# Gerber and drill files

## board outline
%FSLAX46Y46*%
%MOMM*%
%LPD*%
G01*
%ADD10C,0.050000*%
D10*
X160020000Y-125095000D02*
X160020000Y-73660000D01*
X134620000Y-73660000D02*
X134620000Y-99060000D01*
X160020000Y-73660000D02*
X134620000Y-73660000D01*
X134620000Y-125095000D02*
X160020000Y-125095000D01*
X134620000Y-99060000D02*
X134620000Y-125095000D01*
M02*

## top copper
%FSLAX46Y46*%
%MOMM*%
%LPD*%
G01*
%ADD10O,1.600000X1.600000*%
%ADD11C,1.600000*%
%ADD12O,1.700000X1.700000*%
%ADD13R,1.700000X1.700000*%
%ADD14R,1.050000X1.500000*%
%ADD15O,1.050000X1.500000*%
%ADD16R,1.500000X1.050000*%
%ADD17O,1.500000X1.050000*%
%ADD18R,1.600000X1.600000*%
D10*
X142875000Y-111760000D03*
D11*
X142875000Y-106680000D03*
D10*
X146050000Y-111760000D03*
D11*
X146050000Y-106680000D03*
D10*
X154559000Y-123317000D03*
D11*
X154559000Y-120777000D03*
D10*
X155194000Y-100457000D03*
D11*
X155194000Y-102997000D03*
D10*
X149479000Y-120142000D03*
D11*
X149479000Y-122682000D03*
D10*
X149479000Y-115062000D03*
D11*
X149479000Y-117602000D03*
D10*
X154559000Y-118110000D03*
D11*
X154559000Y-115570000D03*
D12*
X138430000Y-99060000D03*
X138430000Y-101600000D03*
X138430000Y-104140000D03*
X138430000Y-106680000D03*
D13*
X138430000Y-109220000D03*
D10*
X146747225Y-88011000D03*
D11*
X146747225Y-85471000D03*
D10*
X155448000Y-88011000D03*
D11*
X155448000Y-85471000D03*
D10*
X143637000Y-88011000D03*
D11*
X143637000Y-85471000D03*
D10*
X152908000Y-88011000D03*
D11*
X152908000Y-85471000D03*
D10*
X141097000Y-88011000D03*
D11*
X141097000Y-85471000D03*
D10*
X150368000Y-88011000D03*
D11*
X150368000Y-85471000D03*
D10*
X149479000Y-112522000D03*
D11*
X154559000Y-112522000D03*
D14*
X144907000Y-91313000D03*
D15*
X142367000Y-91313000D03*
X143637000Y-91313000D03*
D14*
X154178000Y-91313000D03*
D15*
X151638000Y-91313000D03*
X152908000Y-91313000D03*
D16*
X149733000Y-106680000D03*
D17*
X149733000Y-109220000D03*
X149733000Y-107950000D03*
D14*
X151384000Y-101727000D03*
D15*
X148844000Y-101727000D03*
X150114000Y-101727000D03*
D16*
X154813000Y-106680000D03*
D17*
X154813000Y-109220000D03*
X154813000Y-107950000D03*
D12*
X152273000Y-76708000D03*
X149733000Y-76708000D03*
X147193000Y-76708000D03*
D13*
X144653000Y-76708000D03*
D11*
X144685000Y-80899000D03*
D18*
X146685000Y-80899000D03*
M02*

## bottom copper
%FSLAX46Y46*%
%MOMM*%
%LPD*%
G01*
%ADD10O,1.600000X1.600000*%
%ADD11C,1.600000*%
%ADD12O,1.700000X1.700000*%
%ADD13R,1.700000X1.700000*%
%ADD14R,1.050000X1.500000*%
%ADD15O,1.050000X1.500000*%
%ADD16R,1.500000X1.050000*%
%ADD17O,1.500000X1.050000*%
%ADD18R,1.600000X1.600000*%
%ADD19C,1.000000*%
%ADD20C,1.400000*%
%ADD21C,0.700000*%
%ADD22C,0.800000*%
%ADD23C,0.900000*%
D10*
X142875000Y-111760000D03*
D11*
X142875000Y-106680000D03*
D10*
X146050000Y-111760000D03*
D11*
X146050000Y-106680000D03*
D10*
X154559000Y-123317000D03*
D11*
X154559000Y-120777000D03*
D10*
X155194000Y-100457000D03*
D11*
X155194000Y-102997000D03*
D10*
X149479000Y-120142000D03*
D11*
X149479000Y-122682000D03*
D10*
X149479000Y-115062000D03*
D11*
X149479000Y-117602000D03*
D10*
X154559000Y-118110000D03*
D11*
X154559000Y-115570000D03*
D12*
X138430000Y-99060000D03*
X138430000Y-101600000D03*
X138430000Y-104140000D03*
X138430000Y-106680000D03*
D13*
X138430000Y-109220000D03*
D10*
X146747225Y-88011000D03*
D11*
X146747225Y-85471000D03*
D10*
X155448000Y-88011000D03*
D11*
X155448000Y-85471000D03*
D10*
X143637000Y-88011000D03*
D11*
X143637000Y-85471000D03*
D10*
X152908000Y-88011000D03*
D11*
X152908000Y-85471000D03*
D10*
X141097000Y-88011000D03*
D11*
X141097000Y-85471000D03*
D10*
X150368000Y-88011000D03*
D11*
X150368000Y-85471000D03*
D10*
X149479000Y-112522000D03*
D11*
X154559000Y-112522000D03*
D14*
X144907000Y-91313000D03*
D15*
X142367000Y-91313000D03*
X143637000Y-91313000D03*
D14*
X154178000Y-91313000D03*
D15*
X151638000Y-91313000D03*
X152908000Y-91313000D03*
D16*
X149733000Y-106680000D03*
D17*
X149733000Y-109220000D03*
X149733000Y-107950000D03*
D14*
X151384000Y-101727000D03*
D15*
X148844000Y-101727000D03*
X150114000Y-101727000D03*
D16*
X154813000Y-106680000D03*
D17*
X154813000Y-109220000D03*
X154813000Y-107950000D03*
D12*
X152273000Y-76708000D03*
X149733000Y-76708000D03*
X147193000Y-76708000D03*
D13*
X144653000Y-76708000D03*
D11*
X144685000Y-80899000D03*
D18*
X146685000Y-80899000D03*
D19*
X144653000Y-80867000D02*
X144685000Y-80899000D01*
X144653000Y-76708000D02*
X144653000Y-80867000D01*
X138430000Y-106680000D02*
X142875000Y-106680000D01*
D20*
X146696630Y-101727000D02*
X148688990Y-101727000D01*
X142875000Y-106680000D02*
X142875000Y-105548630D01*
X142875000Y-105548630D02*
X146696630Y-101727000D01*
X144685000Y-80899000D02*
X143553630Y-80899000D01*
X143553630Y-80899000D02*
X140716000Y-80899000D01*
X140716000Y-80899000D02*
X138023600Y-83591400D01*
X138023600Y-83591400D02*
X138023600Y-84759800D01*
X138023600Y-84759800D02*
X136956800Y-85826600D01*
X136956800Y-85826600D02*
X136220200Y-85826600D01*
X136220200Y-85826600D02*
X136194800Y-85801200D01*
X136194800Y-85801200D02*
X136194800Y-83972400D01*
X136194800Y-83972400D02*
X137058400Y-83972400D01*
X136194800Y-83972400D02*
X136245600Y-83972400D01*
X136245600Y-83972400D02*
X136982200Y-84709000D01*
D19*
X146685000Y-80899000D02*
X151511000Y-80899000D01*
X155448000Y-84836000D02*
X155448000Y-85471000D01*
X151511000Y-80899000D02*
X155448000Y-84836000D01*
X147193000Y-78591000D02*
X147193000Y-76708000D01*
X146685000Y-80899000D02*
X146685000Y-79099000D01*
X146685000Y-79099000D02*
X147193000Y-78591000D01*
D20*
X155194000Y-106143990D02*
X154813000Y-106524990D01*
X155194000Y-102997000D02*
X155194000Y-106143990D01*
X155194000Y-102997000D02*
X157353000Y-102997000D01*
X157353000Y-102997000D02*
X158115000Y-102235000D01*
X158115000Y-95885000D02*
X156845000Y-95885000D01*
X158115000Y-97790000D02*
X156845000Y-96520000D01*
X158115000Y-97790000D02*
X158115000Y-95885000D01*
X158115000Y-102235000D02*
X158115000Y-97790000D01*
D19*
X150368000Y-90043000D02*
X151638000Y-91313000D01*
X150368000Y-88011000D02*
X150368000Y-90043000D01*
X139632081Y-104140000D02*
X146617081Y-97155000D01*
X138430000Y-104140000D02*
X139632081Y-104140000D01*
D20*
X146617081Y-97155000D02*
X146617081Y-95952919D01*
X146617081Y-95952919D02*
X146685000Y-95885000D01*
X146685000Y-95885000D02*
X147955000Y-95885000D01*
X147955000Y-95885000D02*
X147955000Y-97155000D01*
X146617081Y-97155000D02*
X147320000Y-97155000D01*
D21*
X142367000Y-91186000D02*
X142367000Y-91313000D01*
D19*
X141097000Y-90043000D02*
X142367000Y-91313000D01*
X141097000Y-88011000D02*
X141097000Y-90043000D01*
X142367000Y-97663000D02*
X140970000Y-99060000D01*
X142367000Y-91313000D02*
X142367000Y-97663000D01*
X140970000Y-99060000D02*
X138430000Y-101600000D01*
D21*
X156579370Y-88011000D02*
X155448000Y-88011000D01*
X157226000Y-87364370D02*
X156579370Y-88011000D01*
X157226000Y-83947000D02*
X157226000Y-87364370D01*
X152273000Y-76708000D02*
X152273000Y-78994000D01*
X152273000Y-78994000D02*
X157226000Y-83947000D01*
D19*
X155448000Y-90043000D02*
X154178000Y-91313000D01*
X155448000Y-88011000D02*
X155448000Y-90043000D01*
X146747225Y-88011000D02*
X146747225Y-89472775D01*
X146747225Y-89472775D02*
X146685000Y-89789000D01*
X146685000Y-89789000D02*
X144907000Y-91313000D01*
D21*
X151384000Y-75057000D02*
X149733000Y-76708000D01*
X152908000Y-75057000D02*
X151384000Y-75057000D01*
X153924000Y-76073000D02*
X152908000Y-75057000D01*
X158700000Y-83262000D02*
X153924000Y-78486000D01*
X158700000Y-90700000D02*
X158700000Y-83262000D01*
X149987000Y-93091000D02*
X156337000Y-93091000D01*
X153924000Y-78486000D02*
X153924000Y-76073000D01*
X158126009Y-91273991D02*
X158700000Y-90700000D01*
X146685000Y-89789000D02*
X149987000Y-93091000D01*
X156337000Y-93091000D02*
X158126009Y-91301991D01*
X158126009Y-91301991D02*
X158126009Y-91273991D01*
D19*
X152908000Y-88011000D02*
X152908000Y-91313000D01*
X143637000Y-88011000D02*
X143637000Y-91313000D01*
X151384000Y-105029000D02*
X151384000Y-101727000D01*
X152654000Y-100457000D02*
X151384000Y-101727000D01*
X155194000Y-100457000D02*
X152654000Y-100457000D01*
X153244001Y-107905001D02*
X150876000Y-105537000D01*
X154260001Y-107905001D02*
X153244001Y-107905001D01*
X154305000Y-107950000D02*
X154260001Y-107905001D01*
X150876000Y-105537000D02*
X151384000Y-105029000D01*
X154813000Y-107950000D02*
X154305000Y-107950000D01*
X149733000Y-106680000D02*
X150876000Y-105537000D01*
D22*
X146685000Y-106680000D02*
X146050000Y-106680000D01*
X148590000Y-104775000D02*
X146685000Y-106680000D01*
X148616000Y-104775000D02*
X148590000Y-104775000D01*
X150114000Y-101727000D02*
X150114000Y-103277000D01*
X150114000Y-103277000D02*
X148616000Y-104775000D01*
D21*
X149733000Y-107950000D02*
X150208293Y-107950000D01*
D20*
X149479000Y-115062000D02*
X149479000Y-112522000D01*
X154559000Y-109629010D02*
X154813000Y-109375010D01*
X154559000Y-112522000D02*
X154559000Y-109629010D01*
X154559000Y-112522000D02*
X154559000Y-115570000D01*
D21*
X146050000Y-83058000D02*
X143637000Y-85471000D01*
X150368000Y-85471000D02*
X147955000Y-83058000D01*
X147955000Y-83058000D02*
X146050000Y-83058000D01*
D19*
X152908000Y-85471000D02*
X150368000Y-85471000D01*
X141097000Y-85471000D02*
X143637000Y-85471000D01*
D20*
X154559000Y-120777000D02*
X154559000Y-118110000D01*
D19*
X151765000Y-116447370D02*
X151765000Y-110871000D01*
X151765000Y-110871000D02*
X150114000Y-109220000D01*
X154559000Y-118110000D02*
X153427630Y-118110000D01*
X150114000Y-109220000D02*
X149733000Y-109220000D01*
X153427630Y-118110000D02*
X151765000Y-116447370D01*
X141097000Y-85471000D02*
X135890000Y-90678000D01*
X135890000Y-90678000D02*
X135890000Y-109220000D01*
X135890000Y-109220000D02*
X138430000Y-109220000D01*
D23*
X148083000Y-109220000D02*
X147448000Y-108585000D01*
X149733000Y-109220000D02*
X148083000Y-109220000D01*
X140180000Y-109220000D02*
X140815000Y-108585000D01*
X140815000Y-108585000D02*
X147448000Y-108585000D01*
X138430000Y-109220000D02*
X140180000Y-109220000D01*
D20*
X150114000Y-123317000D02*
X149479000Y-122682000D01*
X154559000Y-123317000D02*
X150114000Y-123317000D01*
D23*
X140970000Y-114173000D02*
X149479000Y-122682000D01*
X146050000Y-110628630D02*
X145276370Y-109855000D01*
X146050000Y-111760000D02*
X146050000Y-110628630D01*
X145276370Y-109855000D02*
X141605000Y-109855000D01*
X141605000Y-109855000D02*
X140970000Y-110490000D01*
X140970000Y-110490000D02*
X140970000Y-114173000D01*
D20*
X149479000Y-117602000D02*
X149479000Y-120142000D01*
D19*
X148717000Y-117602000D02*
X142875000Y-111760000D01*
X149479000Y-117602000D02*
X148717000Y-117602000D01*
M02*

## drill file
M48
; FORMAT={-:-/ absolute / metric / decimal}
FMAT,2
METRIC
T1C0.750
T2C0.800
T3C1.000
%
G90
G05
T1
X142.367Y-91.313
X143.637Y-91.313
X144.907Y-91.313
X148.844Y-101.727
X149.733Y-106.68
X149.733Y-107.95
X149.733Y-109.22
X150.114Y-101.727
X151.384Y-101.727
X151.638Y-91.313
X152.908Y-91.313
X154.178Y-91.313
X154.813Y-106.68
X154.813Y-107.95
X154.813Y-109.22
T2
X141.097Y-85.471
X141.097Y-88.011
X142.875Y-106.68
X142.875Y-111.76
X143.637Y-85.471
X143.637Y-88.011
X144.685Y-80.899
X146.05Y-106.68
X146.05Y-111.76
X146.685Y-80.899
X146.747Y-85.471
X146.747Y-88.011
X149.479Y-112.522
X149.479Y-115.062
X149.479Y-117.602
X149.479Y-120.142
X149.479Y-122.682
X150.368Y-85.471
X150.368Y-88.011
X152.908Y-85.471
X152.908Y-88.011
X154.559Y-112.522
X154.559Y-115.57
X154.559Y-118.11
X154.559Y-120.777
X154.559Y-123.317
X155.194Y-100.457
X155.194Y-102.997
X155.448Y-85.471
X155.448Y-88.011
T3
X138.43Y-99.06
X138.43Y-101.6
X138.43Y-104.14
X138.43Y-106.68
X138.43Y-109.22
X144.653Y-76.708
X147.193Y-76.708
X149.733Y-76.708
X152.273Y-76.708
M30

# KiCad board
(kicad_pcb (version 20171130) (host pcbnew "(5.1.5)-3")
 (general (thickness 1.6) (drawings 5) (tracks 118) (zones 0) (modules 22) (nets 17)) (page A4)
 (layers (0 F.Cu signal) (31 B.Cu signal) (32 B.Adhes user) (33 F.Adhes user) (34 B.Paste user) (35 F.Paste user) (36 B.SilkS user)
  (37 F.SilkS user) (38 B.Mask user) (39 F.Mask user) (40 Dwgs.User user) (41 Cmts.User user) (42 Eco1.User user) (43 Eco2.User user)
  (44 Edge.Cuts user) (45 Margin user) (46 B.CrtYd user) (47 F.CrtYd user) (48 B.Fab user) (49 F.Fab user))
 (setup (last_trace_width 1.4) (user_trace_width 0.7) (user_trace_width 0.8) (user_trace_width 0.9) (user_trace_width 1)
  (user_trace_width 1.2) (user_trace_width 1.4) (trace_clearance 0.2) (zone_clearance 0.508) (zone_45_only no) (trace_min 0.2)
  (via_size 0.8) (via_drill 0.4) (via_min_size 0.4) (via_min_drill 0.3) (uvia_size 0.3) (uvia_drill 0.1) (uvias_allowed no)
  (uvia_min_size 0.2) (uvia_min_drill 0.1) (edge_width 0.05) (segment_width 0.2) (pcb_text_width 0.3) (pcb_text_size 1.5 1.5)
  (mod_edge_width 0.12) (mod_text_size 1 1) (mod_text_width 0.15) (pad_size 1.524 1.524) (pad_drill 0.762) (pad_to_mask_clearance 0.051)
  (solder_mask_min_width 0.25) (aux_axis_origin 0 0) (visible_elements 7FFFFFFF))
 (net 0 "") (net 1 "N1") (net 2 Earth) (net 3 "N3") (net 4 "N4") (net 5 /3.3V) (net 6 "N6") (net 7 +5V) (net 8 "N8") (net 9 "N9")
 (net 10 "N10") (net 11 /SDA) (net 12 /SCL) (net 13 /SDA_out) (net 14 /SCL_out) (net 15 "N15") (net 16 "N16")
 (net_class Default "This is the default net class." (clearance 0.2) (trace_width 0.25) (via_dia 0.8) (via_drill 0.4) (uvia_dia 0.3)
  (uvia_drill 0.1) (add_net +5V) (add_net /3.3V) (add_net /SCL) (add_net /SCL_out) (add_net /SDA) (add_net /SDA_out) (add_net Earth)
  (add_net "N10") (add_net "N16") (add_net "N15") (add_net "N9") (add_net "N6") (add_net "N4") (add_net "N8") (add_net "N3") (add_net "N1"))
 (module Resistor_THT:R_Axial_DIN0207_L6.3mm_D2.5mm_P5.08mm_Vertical (layer F.Cu) (at 142.875 106.68 270)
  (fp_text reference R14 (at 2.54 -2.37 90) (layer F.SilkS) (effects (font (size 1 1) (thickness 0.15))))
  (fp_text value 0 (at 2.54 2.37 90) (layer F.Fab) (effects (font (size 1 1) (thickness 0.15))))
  (pad 2 thru_hole oval (at 5.08 0 270) (size 1.6 1.6) (drill 0.8) (layers *.Cu *.Mask) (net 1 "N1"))
  (pad 1 thru_hole circle (at 0 0 270) (size 1.6 1.6) (drill 0.8) (layers *.Cu *.Mask) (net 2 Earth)))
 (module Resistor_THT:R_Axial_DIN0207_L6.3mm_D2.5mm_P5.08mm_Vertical (layer F.Cu) (at 146.05 106.68 270)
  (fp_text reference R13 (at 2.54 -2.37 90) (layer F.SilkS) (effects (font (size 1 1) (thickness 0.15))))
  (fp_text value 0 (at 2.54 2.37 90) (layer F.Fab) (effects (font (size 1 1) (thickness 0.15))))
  (pad 2 thru_hole oval (at 5.08 0 270) (size 1.6 1.6) (drill 0.8) (layers *.Cu *.Mask) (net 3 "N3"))
  (pad 1 thru_hole circle (at 0 0 270) (size 1.6 1.6) (drill 0.8) (layers *.Cu *.Mask) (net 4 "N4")))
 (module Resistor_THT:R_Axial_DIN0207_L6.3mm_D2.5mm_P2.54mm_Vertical (layer F.Cu) (at 154.559 120.777 270)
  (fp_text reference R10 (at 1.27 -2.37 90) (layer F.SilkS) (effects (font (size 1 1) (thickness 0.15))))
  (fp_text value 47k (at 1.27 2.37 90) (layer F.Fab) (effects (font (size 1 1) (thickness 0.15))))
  (pad 2 thru_hole oval (at 2.54 0 270) (size 1.6 1.6) (drill 0.8) (layers *.Cu *.Mask) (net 3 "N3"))
  (pad 1 thru_hole circle (at 0 0 270) (size 1.6 1.6) (drill 0.8) (layers *.Cu *.Mask) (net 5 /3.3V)))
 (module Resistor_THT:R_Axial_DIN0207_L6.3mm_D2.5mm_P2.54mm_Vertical (layer F.Cu) (at 155.194 102.997 90)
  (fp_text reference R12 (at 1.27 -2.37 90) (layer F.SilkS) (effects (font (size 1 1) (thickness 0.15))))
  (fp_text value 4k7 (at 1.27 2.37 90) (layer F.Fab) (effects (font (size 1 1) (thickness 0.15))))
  (pad 2 thru_hole oval (at 2.54 0 90) (size 1.6 1.6) (drill 0.8) (layers *.Cu *.Mask) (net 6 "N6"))
  (pad 1 thru_hole circle (at 0 0 90) (size 1.6 1.6) (drill 0.8) (layers *.Cu *.Mask) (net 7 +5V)))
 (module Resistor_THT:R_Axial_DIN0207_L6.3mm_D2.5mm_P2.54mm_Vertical (layer F.Cu) (at 149.479 122.682 90)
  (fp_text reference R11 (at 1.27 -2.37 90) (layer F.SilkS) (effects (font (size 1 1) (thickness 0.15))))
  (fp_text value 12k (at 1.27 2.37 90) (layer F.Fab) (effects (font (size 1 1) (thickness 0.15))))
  (pad 2 thru_hole oval (at 2.54 0 90) (size 1.6 1.6) (drill 0.8) (layers *.Cu *.Mask) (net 1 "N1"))
  (pad 1 thru_hole circle (at 0 0 90) (size 1.6 1.6) (drill 0.8) (layers *.Cu *.Mask) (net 3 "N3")))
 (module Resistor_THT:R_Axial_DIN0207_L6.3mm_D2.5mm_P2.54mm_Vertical (layer F.Cu) (at 149.479 117.602 90)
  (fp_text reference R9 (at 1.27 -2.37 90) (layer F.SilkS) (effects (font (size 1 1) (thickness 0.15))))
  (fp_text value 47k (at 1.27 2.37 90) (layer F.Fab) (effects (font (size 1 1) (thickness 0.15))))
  (pad 2 thru_hole oval (at 2.54 0 90) (size 1.6 1.6) (drill 0.8) (layers *.Cu *.Mask) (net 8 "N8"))
  (pad 1 thru_hole circle (at 0 0 90) (size 1.6 1.6) (drill 0.8) (layers *.Cu *.Mask) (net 1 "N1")))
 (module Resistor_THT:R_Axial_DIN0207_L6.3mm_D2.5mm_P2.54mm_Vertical (layer F.Cu) (at 154.559 115.57 270)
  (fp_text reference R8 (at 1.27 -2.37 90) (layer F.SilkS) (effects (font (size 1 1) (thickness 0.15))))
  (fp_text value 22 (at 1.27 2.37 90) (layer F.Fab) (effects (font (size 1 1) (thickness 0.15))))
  (pad 2 thru_hole oval (at 2.54 0 270) (size 1.6 1.6) (drill 0.8) (layers *.Cu *.Mask) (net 5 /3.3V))
  (pad 1 thru_hole circle (at 0 0 270) (size 1.6 1.6) (drill 0.8) (layers *.Cu *.Mask) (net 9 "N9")))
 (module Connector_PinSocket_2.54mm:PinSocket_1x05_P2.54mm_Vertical (layer F.Cu) (at 138.43 109.22 180)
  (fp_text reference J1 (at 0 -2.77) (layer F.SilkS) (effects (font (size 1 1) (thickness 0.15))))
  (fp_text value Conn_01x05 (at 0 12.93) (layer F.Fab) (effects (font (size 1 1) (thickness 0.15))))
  (pad 5 thru_hole oval (at 0 10.16 180) (size 1.7 1.7) (drill 1) (layers *.Cu *.Mask) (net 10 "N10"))
  (pad 4 thru_hole oval (at 0 7.62 180) (size 1.7 1.7) (drill 1) (layers *.Cu *.Mask) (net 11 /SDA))
  (pad 3 thru_hole oval (at 0 5.08 180) (size 1.7 1.7) (drill 1) (layers *.Cu *.Mask) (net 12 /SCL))
  (pad 2 thru_hole oval (at 0 2.54 180) (size 1.7 1.7) (drill 1) (layers *.Cu *.Mask) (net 2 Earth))
  (pad 1 thru_hole rect (at 0 0 180) (size 1.7 1.7) (drill 1) (layers *.Cu *.Mask) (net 5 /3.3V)))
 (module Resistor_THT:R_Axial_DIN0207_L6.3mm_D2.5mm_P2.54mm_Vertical (layer F.Cu) (at 146.747225 85.471 270)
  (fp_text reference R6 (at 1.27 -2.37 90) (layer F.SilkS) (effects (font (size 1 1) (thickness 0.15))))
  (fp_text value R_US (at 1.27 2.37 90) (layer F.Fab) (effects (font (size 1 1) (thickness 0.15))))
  (pad 2 thru_hole oval (at 2.54 0 270) (size 1.6 1.6) (drill 0.8) (layers *.Cu *.Mask) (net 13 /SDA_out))
  (pad 1 thru_hole circle (at 0 0 270) (size 1.6 1.6) (drill 0.8) (layers *.Cu *.Mask) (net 7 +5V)))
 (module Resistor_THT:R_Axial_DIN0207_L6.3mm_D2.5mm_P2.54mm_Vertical (layer F.Cu) (at 155.448 85.471 270)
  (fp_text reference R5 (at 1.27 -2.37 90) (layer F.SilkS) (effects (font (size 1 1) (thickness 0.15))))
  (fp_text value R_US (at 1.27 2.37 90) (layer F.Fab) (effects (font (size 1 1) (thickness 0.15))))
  (pad 2 thru_hole oval (at 2.54 0 270) (size 1.6 1.6) (drill 0.8) (layers *.Cu *.Mask) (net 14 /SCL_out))
  (pad 1 thru_hole circle (at 0 0 270) (size 1.6 1.6) (drill 0.8) (layers *.Cu *.Mask) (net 7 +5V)))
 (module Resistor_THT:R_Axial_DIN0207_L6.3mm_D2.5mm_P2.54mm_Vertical (layer F.Cu) (at 143.637 85.471 270)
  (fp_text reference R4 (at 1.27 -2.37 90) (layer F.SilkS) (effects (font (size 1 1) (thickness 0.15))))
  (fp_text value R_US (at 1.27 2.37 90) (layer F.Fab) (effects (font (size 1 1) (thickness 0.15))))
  (pad 2 thru_hole oval (at 2.54 0 270) (size 1.6 1.6) (drill 0.8) (layers *.Cu *.Mask) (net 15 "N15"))
  (pad 1 thru_hole circle (at 0 0 270) (size 1.6 1.6) (drill 0.8) (layers *.Cu *.Mask) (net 5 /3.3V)))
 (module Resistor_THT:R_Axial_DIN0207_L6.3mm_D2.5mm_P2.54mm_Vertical (layer F.Cu) (at 152.908 85.471 270)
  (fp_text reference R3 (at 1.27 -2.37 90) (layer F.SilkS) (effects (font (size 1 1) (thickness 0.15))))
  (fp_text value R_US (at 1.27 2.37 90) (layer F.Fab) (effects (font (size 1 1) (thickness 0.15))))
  (pad 2 thru_hole oval (at 2.54 0 270) (size 1.6 1.6) (drill 0.8) (layers *.Cu *.Mask) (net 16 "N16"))
  (pad 1 thru_hole circle (at 0 0 270) (size 1.6 1.6) (drill 0.8) (layers *.Cu *.Mask) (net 5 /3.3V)))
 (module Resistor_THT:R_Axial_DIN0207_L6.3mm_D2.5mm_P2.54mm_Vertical (layer F.Cu) (at 141.097 85.471 270)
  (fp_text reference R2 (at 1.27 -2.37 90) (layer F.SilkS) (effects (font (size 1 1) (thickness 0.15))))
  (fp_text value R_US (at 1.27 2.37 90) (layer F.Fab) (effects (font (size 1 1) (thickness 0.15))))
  (pad 2 thru_hole oval (at 2.54 0 270) (size 1.6 1.6) (drill 0.8) (layers *.Cu *.Mask) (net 11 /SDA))
  (pad 1 thru_hole circle (at 0 0 270) (size 1.6 1.6) (drill 0.8) (layers *.Cu *.Mask) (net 5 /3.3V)))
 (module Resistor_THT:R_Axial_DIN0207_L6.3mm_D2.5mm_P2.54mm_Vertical (layer F.Cu) (at 150.368 85.471 270)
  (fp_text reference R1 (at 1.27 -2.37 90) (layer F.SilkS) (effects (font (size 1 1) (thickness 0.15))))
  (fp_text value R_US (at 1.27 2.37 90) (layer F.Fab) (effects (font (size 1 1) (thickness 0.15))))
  (pad 2 thru_hole oval (at 2.54 0 270) (size 1.6 1.6) (drill 0.8) (layers *.Cu *.Mask) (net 12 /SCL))
  (pad 1 thru_hole circle (at 0 0 270) (size 1.6 1.6) (drill 0.8) (layers *.Cu *.Mask) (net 5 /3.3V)))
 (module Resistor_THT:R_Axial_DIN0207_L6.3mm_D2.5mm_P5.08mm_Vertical (layer F.Cu) (at 154.559 112.522 180)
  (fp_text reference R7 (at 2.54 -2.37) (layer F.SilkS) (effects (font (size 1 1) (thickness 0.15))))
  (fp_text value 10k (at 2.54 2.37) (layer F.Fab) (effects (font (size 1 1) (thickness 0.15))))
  (pad 2 thru_hole oval (at 5.08 0 180) (size 1.6 1.6) (drill 0.8) (layers *.Cu *.Mask) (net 8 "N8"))
  (pad 1 thru_hole circle (at 0 0 180) (size 1.6 1.6) (drill 0.8) (layers *.Cu *.Mask) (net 9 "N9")))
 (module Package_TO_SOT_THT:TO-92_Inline (layer F.Cu) (at 144.907 91.313 180)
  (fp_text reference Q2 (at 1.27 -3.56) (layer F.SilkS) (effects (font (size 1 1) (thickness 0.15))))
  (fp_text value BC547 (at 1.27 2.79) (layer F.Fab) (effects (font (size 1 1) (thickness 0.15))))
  (pad 3 thru_hole rect (at 0 0 180) (size 1.05 1.5) (drill 0.75) (layers *.Cu *.Mask) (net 13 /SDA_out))
  (pad 1 thru_hole oval (at 2.54 0 180) (size 1.05 1.5) (drill 0.75) (layers *.Cu *.Mask) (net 11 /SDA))
  (pad 2 thru_hole oval (at 1.27 0 180) (size 1.05 1.5) (drill 0.75) (layers *.Cu *.Mask) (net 15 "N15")))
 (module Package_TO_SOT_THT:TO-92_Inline (layer F.Cu) (at 154.178 91.313 180)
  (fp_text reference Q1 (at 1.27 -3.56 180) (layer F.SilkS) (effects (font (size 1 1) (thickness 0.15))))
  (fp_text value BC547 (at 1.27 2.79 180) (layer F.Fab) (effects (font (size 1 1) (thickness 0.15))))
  (pad 3 thru_hole rect (at 0 0 180) (size 1.05 1.5) (drill 0.75) (layers *.Cu *.Mask) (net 14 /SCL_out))
  (pad 1 thru_hole oval (at 2.54 0 180) (size 1.05 1.5) (drill 0.75) (layers *.Cu *.Mask) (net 12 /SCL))
  (pad 2 thru_hole oval (at 1.27 0 180) (size 1.05 1.5) (drill 0.75) (layers *.Cu *.Mask) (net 16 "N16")))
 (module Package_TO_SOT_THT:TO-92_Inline (layer F.Cu) (at 149.733 106.68 270)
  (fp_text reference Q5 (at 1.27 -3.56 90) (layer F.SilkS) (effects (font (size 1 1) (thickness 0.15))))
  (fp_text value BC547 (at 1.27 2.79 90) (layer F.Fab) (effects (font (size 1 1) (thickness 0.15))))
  (pad 3 thru_hole rect (at 0 0 270) (size 1.05 1.5) (drill 0.75) (layers *.Cu *.Mask) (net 6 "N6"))
  (pad 1 thru_hole oval (at 2.54 0 270) (size 1.05 1.5) (drill 0.75) (layers *.Cu *.Mask) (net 5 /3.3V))
  (pad 2 thru_hole oval (at 1.27 0 270) (size 1.05 1.5) (drill 0.75) (layers *.Cu *.Mask) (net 8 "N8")))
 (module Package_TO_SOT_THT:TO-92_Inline (layer F.Cu) (at 151.384 101.727 180)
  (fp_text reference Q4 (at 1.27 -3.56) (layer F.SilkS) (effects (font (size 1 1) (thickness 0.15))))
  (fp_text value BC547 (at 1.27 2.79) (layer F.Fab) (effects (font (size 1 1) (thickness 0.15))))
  (pad 3 thru_hole rect (at 0 0 180) (size 1.05 1.5) (drill 0.75) (layers *.Cu *.Mask) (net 6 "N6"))
  (pad 1 thru_hole oval (at 2.54 0 180) (size 1.05 1.5) (drill 0.75) (layers *.Cu *.Mask) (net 2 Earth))
  (pad 2 thru_hole oval (at 1.27 0 180) (size 1.05 1.5) (drill 0.75) (layers *.Cu *.Mask) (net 4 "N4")))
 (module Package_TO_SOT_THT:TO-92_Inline (layer F.Cu) (at 154.813 106.68 270)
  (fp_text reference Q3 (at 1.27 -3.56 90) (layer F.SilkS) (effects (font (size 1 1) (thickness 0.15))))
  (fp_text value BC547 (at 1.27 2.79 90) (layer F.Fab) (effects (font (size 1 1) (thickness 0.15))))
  (pad 3 thru_hole rect (at 0 0 270) (size 1.05 1.5) (drill 0.75) (layers *.Cu *.Mask) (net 7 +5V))
  (pad 1 thru_hole oval (at 2.54 0 270) (size 1.05 1.5) (drill 0.75) (layers *.Cu *.Mask) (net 9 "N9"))
  (pad 2 thru_hole oval (at 1.27 0 270) (size 1.05 1.5) (drill 0.75) (layers *.Cu *.Mask) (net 6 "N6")))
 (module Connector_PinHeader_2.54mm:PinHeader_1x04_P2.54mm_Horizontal (layer F.Cu) (at 144.653 76.708 90)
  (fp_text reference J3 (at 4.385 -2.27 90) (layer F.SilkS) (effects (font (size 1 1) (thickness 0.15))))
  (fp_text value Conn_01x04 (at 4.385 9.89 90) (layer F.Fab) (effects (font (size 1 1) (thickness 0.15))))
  (pad 4 thru_hole oval (at 0 7.62 90) (size 1.7 1.7) (drill 1) (layers *.Cu *.Mask) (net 14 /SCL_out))
  (pad 3 thru_hole oval (at 0 5.08 90) (size 1.7 1.7) (drill 1) (layers *.Cu *.Mask) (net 13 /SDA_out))
  (pad 2 thru_hole oval (at 0 2.54 90) (size 1.7 1.7) (drill 1) (layers *.Cu *.Mask) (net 7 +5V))
  (pad 1 thru_hole rect (at 0 0 90) (size 1.7 1.7) (drill 1) (layers *.Cu *.Mask) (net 2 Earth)))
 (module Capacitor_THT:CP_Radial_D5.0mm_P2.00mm (layer F.Cu) (at 146.685 80.899 180)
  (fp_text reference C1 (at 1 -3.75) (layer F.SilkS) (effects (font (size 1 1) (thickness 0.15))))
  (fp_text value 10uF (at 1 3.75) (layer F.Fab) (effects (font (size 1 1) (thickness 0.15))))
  (pad 2 thru_hole circle (at 2 0 180) (size 1.6 1.6) (drill 0.8) (layers *.Cu *.Mask) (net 2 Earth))
  (pad 1 thru_hole rect (at 0 0 180) (size 1.6 1.6) (drill 0.8) (layers *.Cu *.Mask) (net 7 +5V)))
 (gr_line (start 160.02 125.095) (end 160.02 73.66) (layer Edge.Cuts) (width 0.05))
 (gr_line (start 134.62 73.66) (end 134.62 99.06) (layer Edge.Cuts) (width 0.05))
 (gr_line (start 160.02 73.66) (end 134.62 73.66) (layer Edge.Cuts) (width 0.05))
 (gr_line (start 134.62 125.095) (end 160.02 125.095) (layer Edge.Cuts) (width 0.05))
 (gr_line (start 134.62 99.06) (end 134.62 125.095) (layer Edge.Cuts) (width 0.05))
 (segment (start 144.653 80.867) (end 144.685 80.899) (width 1) (layer B.Cu) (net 2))
 (segment (start 144.653 76.708) (end 144.653 80.867) (width 1) (layer B.Cu) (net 2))
 (segment (start 138.43 106.68) (end 142.875 106.68) (width 1) (layer B.Cu) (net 2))
 (segment (start 146.69663 101.727) (end 148.68899 101.727) (width 1.4) (layer B.Cu) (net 2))
 (segment (start 142.875 106.68) (end 142.875 105.54863) (width 1.4) (layer B.Cu) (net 2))
 (segment (start 142.875 105.54863) (end 146.69663 101.727) (width 1.4) (layer B.Cu) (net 2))
 (segment (start 144.685 80.899) (end 143.55363 80.899) (width 1.4) (layer B.Cu) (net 2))
 (segment (start 143.55363 80.899) (end 140.716 80.899) (width 1.4) (layer B.Cu) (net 2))
 (segment (start 140.716 80.899) (end 138.0236 83.5914) (width 1.4) (layer B.Cu) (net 2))
 (segment (start 138.0236 83.5914) (end 138.0236 84.7598) (width 1.4) (layer B.Cu) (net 2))
 (segment (start 138.0236 84.7598) (end 136.9568 85.8266) (width 1.4) (layer B.Cu) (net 2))
 (segment (start 136.9568 85.8266) (end 136.2202 85.8266) (width 1.4) (layer B.Cu) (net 2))
 (segment (start 136.2202 85.8266) (end 136.1948 85.8012) (width 1.4) (layer B.Cu) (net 2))
 (segment (start 136.1948 85.8012) (end 136.1948 83.9724) (width 1.4) (layer B.Cu) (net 2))
 (segment (start 136.1948 83.9724) (end 137.0584 83.9724) (width 1.4) (layer B.Cu) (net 2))
 (segment (start 136.1948 83.9724) (end 136.2456 83.9724) (width 1.4) (layer B.Cu) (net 2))
 (segment (start 136.2456 83.9724) (end 136.9822 84.709) (width 1.4) (layer B.Cu) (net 2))
 (segment (start 146.685 80.899) (end 151.511 80.899) (width 1) (layer B.Cu) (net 7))
 (segment (start 155.448 84.836) (end 155.448 85.471) (width 1) (layer B.Cu) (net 7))
 (segment (start 151.511 80.899) (end 155.448 84.836) (width 1) (layer B.Cu) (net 7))
 (segment (start 147.193 78.591) (end 147.193 76.708) (width 1) (layer B.Cu) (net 7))
 (segment (start 146.685 80.899) (end 146.685 79.099) (width 1) (layer B.Cu) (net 7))
 (segment (start 146.685 79.099) (end 147.193 78.591) (width 1) (layer B.Cu) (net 7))
 (segment (start 155.194 106.14399) (end 154.813 106.52499) (width 1.4) (layer B.Cu) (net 7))
 (segment (start 155.194 102.997) (end 155.194 106.14399) (width 1.4) (layer B.Cu) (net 7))
 (segment (start 155.194 102.997) (end 157.353 102.997) (width 1.4) (layer B.Cu) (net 7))
 (segment (start 157.353 102.997) (end 158.115 102.235) (width 1.4) (layer B.Cu) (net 7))
 (segment (start 158.115 95.885) (end 156.845 95.885) (width 1.4) (layer B.Cu) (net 7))
 (segment (start 158.115 97.79) (end 156.845 96.52) (width 1.4) (layer B.Cu) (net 7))
 (segment (start 158.115 97.79) (end 158.115 95.885) (width 1.4) (layer B.Cu) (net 7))
 (segment (start 158.115 102.235) (end 158.115 97.79) (width 1.4) (layer B.Cu) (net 7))
 (segment (start 150.368 90.043) (end 151.638 91.313) (width 1) (layer B.Cu) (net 12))
 (segment (start 150.368 88.011) (end 150.368 90.043) (width 1) (layer B.Cu) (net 12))
 (segment (start 139.632081 104.14) (end 146.617081 97.155) (width 1) (layer B.Cu) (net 12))
 (segment (start 138.43 104.14) (end 139.632081 104.14) (width 1) (layer B.Cu) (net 12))
 (segment (start 146.617081 97.155) (end 146.617081 95.952919) (width 1.4) (layer B.Cu) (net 12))
 (segment (start 146.617081 95.952919) (end 146.685 95.885) (width 1.4) (layer B.Cu) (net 12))
 (segment (start 146.685 95.885) (end 147.955 95.885) (width 1.4) (layer B.Cu) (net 12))
 (segment (start 147.955 95.885) (end 147.955 97.155) (width 1.4) (layer B.Cu) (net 12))
 (segment (start 146.617081 97.155) (end 147.32 97.155) (width 1.4) (layer B.Cu) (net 12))
 (segment (start 142.367 91.186) (end 142.367 91.313) (width 0.7) (layer B.Cu) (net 11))
 (segment (start 141.097 90.043) (end 142.367 91.313) (width 1) (layer B.Cu) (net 11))
 (segment (start 141.097 88.011) (end 141.097 90.043) (width 1) (layer B.Cu) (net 11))
 (segment (start 142.367 97.663) (end 140.97 99.06) (width 1) (layer B.Cu) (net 11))
 (segment (start 142.367 91.313) (end 142.367 97.663) (width 1) (layer B.Cu) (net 11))
 (segment (start 140.97 99.06) (end 138.43 101.6) (width 1) (layer B.Cu) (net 11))
 (segment (start 156.57937 88.011) (end 155.448 88.011) (width 0.7) (layer B.Cu) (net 14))
 (segment (start 157.226 87.36437) (end 156.57937 88.011) (width 0.7) (layer B.Cu) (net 14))
 (segment (start 157.226 83.947) (end 157.226 87.36437) (width 0.7) (layer B.Cu) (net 14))
 (segment (start 152.273 76.708) (end 152.273 78.994) (width 0.7) (layer B.Cu) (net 14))
 (segment (start 152.273 78.994) (end 157.226 83.947) (width 0.7) (layer B.Cu) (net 14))
 (segment (start 155.448 90.043) (end 154.178 91.313) (width 1) (layer B.Cu) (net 14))
 (segment (start 155.448 88.011) (end 155.448 90.043) (width 1) (layer B.Cu) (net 14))
 (segment (start 146.747225 88.011) (end 146.747225 89.472775) (width 1) (layer B.Cu) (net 13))
 (segment (start 146.747225 89.472775) (end 146.685 89.789) (width 1) (layer B.Cu) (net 13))
 (segment (start 146.685 89.789) (end 144.907 91.313) (width 1) (layer B.Cu) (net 13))
 (segment (start 151.384 75.057) (end 149.733 76.708) (width 0.7) (layer B.Cu) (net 13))
 (segment (start 152.908 75.057) (end 151.384 75.057) (width 0.7) (layer B.Cu) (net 13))
 (segment (start 153.924 76.073) (end 152.908 75.057) (width 0.7) (layer B.Cu) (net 13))
 (segment (start 158.7 83.262) (end 153.924 78.486) (width 0.7) (layer B.Cu) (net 13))
 (segment (start 158.7 90.7) (end 158.7 83.262) (width 0.7) (layer B.Cu) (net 13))
 (segment (start 149.987 93.091) (end 156.337 93.091) (width 0.7) (layer B.Cu) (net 13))
 (segment (start 153.924 78.486) (end 153.924 76.073) (width 0.7) (layer B.Cu) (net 13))
 (segment (start 158.126009 91.273991) (end 158.7 90.7) (width 0.7) (layer B.Cu) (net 13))
 (segment (start 146.685 89.789) (end 149.987 93.091) (width 0.7) (layer B.Cu) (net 13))
 (segment (start 156.337 93.091) (end 158.126009 91.301991) (width 0.7) (layer B.Cu) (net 13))
 (segment (start 158.126009 91.301991) (end 158.126009 91.273991) (width 0.7) (layer B.Cu) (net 13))
 (segment (start 152.908 88.011) (end 152.908 91.313) (width 1) (layer B.Cu) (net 16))
 (segment (start 143.637 88.011) (end 143.637 91.313) (width 1) (layer B.Cu) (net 15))
 (segment (start 151.384 105.029) (end 151.384 101.727) (width 1) (layer B.Cu) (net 6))
 (segment (start 152.654 100.457) (end 151.384 101.727) (width 1) (layer B.Cu) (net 6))
 (segment (start 155.194 100.457) (end 152.654 100.457) (width 1) (layer B.Cu) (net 6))
 (segment (start 153.244001 107.905001) (end 150.876 105.537) (width 1) (layer B.Cu) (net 6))
 (segment (start 154.260001 107.905001) (end 153.244001 107.905001) (width 1) (layer B.Cu) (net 6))
 (segment (start 154.305 107.95) (end 154.260001 107.905001) (width 1) (layer B.Cu) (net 6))
 (segment (start 150.876 105.537) (end 151.384 105.029) (width 1) (layer B.Cu) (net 6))
 (segment (start 154.813 107.95) (end 154.305 107.95) (width 1) (layer B.Cu) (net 6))
 (segment (start 149.733 106.68) (end 150.876 105.537) (width 1) (layer B.Cu) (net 6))
 (segment (start 146.685 106.68) (end 146.05 106.68) (width 0.8) (layer B.Cu) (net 4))
 (segment (start 148.59 104.775) (end 146.685 106.68) (width 0.8) (layer B.Cu) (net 4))
 (segment (start 148.616 104.775) (end 148.59 104.775) (width 0.8) (layer B.Cu) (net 4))
 (segment (start 150.114 101.727) (end 150.114 103.277) (width 0.8) (layer B.Cu) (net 4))
 (segment (start 150.114 103.277) (end 148.616 104.775) (width 0.8) (layer B.Cu) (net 4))
 (segment (start 149.733 107.95) (end 150.208293 107.95) (width 0.7) (layer B.Cu) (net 8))
 (segment (start 149.479 115.062) (end 149.479 112.522) (width 1.4) (layer B.Cu) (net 8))
 (segment (start 154.559 109.62901) (end 154.813 109.37501) (width 1.4) (layer B.Cu) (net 9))
 (segment (start 154.559 112.522) (end 154.559 109.62901) (width 1.4) (layer B.Cu) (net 9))
 (segment (start 154.559 112.522) (end 154.559 115.57) (width 1.4) (layer B.Cu) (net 9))
 (segment (start 146.05 83.058) (end 143.637 85.471) (width 0.7) (layer B.Cu) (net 5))
 (segment (start 150.368 85.471) (end 147.955 83.058) (width 0.7) (layer B.Cu) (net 5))
 (segment (start 147.955 83.058) (end 146.05 83.058) (width 0.7) (layer B.Cu) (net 5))
 (segment (start 152.908 85.471) (end 150.368 85.471) (width 1) (layer B.Cu) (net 5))
 (segment (start 141.097 85.471) (end 143.637 85.471) (width 1) (layer B.Cu) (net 5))
 (segment (start 154.559 120.777) (end 154.559 118.11) (width 1.4) (layer B.Cu) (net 5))
 (segment (start 151.765 116.44737) (end 151.765 110.871) (width 1) (layer B.Cu) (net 5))
 (segment (start 151.765 110.871) (end 150.114 109.22) (width 1) (layer B.Cu) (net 5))
 (segment (start 154.559 118.11) (end 153.42763 118.11) (width 1) (layer B.Cu) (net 5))
 (segment (start 150.114 109.22) (end 149.733 109.22) (width 1) (layer B.Cu) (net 5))
 (segment (start 153.42763 118.11) (end 151.765 116.44737) (width 1) (layer B.Cu) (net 5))
 (segment (start 141.097 85.471) (end 135.89 90.678) (width 1) (layer B.Cu) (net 5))
 (segment (start 135.89 90.678) (end 135.89 109.22) (width 1) (layer B.Cu) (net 5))
 (segment (start 135.89 109.22) (end 138.43 109.22) (width 1) (layer B.Cu) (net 5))
 (segment (start 148.083 109.22) (end 147.448 108.585) (width 0.9) (layer B.Cu) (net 5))
 (segment (start 149.733 109.22) (end 148.083 109.22) (width 0.9) (layer B.Cu) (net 5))
 (segment (start 140.18 109.22) (end 140.815 108.585) (width 0.9) (layer B.Cu) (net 5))
 (segment (start 140.815 108.585) (end 147.448 108.585) (width 0.9) (layer B.Cu) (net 5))
 (segment (start 138.43 109.22) (end 140.18 109.22) (width 0.9) (layer B.Cu) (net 5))
 (segment (start 150.114 123.317) (end 149.479 122.682) (width 1.4) (layer B.Cu) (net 3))
 (segment (start 154.559 123.317) (end 150.114 123.317) (width 1.4) (layer B.Cu) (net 3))
 (segment (start 140.97 114.173) (end 149.479 122.682) (width 0.9) (layer B.Cu) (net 3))
 (segment (start 146.05 110.62863) (end 145.27637 109.855) (width 0.9) (layer B.Cu) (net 3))
 (segment (start 146.05 111.76) (end 146.05 110.62863) (width 0.9) (layer B.Cu) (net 3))
 (segment (start 145.27637 109.855) (end 141.605 109.855) (width 0.9) (layer B.Cu) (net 3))
 (segment (start 141.605 109.855) (end 140.97 110.49) (width 0.9) (layer B.Cu) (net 3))
 (segment (start 140.97 110.49) (end 140.97 114.173) (width 0.9) (layer B.Cu) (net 3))
 (segment (start 149.479 117.602) (end 149.479 120.142) (width 1.4) (layer B.Cu) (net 1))
 (segment (start 148.717 117.602) (end 142.875 111.76) (width 1) (layer B.Cu) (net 1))
 (segment (start 149.479 117.602) (end 148.717 117.602) (width 1) (layer B.Cu) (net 1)))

